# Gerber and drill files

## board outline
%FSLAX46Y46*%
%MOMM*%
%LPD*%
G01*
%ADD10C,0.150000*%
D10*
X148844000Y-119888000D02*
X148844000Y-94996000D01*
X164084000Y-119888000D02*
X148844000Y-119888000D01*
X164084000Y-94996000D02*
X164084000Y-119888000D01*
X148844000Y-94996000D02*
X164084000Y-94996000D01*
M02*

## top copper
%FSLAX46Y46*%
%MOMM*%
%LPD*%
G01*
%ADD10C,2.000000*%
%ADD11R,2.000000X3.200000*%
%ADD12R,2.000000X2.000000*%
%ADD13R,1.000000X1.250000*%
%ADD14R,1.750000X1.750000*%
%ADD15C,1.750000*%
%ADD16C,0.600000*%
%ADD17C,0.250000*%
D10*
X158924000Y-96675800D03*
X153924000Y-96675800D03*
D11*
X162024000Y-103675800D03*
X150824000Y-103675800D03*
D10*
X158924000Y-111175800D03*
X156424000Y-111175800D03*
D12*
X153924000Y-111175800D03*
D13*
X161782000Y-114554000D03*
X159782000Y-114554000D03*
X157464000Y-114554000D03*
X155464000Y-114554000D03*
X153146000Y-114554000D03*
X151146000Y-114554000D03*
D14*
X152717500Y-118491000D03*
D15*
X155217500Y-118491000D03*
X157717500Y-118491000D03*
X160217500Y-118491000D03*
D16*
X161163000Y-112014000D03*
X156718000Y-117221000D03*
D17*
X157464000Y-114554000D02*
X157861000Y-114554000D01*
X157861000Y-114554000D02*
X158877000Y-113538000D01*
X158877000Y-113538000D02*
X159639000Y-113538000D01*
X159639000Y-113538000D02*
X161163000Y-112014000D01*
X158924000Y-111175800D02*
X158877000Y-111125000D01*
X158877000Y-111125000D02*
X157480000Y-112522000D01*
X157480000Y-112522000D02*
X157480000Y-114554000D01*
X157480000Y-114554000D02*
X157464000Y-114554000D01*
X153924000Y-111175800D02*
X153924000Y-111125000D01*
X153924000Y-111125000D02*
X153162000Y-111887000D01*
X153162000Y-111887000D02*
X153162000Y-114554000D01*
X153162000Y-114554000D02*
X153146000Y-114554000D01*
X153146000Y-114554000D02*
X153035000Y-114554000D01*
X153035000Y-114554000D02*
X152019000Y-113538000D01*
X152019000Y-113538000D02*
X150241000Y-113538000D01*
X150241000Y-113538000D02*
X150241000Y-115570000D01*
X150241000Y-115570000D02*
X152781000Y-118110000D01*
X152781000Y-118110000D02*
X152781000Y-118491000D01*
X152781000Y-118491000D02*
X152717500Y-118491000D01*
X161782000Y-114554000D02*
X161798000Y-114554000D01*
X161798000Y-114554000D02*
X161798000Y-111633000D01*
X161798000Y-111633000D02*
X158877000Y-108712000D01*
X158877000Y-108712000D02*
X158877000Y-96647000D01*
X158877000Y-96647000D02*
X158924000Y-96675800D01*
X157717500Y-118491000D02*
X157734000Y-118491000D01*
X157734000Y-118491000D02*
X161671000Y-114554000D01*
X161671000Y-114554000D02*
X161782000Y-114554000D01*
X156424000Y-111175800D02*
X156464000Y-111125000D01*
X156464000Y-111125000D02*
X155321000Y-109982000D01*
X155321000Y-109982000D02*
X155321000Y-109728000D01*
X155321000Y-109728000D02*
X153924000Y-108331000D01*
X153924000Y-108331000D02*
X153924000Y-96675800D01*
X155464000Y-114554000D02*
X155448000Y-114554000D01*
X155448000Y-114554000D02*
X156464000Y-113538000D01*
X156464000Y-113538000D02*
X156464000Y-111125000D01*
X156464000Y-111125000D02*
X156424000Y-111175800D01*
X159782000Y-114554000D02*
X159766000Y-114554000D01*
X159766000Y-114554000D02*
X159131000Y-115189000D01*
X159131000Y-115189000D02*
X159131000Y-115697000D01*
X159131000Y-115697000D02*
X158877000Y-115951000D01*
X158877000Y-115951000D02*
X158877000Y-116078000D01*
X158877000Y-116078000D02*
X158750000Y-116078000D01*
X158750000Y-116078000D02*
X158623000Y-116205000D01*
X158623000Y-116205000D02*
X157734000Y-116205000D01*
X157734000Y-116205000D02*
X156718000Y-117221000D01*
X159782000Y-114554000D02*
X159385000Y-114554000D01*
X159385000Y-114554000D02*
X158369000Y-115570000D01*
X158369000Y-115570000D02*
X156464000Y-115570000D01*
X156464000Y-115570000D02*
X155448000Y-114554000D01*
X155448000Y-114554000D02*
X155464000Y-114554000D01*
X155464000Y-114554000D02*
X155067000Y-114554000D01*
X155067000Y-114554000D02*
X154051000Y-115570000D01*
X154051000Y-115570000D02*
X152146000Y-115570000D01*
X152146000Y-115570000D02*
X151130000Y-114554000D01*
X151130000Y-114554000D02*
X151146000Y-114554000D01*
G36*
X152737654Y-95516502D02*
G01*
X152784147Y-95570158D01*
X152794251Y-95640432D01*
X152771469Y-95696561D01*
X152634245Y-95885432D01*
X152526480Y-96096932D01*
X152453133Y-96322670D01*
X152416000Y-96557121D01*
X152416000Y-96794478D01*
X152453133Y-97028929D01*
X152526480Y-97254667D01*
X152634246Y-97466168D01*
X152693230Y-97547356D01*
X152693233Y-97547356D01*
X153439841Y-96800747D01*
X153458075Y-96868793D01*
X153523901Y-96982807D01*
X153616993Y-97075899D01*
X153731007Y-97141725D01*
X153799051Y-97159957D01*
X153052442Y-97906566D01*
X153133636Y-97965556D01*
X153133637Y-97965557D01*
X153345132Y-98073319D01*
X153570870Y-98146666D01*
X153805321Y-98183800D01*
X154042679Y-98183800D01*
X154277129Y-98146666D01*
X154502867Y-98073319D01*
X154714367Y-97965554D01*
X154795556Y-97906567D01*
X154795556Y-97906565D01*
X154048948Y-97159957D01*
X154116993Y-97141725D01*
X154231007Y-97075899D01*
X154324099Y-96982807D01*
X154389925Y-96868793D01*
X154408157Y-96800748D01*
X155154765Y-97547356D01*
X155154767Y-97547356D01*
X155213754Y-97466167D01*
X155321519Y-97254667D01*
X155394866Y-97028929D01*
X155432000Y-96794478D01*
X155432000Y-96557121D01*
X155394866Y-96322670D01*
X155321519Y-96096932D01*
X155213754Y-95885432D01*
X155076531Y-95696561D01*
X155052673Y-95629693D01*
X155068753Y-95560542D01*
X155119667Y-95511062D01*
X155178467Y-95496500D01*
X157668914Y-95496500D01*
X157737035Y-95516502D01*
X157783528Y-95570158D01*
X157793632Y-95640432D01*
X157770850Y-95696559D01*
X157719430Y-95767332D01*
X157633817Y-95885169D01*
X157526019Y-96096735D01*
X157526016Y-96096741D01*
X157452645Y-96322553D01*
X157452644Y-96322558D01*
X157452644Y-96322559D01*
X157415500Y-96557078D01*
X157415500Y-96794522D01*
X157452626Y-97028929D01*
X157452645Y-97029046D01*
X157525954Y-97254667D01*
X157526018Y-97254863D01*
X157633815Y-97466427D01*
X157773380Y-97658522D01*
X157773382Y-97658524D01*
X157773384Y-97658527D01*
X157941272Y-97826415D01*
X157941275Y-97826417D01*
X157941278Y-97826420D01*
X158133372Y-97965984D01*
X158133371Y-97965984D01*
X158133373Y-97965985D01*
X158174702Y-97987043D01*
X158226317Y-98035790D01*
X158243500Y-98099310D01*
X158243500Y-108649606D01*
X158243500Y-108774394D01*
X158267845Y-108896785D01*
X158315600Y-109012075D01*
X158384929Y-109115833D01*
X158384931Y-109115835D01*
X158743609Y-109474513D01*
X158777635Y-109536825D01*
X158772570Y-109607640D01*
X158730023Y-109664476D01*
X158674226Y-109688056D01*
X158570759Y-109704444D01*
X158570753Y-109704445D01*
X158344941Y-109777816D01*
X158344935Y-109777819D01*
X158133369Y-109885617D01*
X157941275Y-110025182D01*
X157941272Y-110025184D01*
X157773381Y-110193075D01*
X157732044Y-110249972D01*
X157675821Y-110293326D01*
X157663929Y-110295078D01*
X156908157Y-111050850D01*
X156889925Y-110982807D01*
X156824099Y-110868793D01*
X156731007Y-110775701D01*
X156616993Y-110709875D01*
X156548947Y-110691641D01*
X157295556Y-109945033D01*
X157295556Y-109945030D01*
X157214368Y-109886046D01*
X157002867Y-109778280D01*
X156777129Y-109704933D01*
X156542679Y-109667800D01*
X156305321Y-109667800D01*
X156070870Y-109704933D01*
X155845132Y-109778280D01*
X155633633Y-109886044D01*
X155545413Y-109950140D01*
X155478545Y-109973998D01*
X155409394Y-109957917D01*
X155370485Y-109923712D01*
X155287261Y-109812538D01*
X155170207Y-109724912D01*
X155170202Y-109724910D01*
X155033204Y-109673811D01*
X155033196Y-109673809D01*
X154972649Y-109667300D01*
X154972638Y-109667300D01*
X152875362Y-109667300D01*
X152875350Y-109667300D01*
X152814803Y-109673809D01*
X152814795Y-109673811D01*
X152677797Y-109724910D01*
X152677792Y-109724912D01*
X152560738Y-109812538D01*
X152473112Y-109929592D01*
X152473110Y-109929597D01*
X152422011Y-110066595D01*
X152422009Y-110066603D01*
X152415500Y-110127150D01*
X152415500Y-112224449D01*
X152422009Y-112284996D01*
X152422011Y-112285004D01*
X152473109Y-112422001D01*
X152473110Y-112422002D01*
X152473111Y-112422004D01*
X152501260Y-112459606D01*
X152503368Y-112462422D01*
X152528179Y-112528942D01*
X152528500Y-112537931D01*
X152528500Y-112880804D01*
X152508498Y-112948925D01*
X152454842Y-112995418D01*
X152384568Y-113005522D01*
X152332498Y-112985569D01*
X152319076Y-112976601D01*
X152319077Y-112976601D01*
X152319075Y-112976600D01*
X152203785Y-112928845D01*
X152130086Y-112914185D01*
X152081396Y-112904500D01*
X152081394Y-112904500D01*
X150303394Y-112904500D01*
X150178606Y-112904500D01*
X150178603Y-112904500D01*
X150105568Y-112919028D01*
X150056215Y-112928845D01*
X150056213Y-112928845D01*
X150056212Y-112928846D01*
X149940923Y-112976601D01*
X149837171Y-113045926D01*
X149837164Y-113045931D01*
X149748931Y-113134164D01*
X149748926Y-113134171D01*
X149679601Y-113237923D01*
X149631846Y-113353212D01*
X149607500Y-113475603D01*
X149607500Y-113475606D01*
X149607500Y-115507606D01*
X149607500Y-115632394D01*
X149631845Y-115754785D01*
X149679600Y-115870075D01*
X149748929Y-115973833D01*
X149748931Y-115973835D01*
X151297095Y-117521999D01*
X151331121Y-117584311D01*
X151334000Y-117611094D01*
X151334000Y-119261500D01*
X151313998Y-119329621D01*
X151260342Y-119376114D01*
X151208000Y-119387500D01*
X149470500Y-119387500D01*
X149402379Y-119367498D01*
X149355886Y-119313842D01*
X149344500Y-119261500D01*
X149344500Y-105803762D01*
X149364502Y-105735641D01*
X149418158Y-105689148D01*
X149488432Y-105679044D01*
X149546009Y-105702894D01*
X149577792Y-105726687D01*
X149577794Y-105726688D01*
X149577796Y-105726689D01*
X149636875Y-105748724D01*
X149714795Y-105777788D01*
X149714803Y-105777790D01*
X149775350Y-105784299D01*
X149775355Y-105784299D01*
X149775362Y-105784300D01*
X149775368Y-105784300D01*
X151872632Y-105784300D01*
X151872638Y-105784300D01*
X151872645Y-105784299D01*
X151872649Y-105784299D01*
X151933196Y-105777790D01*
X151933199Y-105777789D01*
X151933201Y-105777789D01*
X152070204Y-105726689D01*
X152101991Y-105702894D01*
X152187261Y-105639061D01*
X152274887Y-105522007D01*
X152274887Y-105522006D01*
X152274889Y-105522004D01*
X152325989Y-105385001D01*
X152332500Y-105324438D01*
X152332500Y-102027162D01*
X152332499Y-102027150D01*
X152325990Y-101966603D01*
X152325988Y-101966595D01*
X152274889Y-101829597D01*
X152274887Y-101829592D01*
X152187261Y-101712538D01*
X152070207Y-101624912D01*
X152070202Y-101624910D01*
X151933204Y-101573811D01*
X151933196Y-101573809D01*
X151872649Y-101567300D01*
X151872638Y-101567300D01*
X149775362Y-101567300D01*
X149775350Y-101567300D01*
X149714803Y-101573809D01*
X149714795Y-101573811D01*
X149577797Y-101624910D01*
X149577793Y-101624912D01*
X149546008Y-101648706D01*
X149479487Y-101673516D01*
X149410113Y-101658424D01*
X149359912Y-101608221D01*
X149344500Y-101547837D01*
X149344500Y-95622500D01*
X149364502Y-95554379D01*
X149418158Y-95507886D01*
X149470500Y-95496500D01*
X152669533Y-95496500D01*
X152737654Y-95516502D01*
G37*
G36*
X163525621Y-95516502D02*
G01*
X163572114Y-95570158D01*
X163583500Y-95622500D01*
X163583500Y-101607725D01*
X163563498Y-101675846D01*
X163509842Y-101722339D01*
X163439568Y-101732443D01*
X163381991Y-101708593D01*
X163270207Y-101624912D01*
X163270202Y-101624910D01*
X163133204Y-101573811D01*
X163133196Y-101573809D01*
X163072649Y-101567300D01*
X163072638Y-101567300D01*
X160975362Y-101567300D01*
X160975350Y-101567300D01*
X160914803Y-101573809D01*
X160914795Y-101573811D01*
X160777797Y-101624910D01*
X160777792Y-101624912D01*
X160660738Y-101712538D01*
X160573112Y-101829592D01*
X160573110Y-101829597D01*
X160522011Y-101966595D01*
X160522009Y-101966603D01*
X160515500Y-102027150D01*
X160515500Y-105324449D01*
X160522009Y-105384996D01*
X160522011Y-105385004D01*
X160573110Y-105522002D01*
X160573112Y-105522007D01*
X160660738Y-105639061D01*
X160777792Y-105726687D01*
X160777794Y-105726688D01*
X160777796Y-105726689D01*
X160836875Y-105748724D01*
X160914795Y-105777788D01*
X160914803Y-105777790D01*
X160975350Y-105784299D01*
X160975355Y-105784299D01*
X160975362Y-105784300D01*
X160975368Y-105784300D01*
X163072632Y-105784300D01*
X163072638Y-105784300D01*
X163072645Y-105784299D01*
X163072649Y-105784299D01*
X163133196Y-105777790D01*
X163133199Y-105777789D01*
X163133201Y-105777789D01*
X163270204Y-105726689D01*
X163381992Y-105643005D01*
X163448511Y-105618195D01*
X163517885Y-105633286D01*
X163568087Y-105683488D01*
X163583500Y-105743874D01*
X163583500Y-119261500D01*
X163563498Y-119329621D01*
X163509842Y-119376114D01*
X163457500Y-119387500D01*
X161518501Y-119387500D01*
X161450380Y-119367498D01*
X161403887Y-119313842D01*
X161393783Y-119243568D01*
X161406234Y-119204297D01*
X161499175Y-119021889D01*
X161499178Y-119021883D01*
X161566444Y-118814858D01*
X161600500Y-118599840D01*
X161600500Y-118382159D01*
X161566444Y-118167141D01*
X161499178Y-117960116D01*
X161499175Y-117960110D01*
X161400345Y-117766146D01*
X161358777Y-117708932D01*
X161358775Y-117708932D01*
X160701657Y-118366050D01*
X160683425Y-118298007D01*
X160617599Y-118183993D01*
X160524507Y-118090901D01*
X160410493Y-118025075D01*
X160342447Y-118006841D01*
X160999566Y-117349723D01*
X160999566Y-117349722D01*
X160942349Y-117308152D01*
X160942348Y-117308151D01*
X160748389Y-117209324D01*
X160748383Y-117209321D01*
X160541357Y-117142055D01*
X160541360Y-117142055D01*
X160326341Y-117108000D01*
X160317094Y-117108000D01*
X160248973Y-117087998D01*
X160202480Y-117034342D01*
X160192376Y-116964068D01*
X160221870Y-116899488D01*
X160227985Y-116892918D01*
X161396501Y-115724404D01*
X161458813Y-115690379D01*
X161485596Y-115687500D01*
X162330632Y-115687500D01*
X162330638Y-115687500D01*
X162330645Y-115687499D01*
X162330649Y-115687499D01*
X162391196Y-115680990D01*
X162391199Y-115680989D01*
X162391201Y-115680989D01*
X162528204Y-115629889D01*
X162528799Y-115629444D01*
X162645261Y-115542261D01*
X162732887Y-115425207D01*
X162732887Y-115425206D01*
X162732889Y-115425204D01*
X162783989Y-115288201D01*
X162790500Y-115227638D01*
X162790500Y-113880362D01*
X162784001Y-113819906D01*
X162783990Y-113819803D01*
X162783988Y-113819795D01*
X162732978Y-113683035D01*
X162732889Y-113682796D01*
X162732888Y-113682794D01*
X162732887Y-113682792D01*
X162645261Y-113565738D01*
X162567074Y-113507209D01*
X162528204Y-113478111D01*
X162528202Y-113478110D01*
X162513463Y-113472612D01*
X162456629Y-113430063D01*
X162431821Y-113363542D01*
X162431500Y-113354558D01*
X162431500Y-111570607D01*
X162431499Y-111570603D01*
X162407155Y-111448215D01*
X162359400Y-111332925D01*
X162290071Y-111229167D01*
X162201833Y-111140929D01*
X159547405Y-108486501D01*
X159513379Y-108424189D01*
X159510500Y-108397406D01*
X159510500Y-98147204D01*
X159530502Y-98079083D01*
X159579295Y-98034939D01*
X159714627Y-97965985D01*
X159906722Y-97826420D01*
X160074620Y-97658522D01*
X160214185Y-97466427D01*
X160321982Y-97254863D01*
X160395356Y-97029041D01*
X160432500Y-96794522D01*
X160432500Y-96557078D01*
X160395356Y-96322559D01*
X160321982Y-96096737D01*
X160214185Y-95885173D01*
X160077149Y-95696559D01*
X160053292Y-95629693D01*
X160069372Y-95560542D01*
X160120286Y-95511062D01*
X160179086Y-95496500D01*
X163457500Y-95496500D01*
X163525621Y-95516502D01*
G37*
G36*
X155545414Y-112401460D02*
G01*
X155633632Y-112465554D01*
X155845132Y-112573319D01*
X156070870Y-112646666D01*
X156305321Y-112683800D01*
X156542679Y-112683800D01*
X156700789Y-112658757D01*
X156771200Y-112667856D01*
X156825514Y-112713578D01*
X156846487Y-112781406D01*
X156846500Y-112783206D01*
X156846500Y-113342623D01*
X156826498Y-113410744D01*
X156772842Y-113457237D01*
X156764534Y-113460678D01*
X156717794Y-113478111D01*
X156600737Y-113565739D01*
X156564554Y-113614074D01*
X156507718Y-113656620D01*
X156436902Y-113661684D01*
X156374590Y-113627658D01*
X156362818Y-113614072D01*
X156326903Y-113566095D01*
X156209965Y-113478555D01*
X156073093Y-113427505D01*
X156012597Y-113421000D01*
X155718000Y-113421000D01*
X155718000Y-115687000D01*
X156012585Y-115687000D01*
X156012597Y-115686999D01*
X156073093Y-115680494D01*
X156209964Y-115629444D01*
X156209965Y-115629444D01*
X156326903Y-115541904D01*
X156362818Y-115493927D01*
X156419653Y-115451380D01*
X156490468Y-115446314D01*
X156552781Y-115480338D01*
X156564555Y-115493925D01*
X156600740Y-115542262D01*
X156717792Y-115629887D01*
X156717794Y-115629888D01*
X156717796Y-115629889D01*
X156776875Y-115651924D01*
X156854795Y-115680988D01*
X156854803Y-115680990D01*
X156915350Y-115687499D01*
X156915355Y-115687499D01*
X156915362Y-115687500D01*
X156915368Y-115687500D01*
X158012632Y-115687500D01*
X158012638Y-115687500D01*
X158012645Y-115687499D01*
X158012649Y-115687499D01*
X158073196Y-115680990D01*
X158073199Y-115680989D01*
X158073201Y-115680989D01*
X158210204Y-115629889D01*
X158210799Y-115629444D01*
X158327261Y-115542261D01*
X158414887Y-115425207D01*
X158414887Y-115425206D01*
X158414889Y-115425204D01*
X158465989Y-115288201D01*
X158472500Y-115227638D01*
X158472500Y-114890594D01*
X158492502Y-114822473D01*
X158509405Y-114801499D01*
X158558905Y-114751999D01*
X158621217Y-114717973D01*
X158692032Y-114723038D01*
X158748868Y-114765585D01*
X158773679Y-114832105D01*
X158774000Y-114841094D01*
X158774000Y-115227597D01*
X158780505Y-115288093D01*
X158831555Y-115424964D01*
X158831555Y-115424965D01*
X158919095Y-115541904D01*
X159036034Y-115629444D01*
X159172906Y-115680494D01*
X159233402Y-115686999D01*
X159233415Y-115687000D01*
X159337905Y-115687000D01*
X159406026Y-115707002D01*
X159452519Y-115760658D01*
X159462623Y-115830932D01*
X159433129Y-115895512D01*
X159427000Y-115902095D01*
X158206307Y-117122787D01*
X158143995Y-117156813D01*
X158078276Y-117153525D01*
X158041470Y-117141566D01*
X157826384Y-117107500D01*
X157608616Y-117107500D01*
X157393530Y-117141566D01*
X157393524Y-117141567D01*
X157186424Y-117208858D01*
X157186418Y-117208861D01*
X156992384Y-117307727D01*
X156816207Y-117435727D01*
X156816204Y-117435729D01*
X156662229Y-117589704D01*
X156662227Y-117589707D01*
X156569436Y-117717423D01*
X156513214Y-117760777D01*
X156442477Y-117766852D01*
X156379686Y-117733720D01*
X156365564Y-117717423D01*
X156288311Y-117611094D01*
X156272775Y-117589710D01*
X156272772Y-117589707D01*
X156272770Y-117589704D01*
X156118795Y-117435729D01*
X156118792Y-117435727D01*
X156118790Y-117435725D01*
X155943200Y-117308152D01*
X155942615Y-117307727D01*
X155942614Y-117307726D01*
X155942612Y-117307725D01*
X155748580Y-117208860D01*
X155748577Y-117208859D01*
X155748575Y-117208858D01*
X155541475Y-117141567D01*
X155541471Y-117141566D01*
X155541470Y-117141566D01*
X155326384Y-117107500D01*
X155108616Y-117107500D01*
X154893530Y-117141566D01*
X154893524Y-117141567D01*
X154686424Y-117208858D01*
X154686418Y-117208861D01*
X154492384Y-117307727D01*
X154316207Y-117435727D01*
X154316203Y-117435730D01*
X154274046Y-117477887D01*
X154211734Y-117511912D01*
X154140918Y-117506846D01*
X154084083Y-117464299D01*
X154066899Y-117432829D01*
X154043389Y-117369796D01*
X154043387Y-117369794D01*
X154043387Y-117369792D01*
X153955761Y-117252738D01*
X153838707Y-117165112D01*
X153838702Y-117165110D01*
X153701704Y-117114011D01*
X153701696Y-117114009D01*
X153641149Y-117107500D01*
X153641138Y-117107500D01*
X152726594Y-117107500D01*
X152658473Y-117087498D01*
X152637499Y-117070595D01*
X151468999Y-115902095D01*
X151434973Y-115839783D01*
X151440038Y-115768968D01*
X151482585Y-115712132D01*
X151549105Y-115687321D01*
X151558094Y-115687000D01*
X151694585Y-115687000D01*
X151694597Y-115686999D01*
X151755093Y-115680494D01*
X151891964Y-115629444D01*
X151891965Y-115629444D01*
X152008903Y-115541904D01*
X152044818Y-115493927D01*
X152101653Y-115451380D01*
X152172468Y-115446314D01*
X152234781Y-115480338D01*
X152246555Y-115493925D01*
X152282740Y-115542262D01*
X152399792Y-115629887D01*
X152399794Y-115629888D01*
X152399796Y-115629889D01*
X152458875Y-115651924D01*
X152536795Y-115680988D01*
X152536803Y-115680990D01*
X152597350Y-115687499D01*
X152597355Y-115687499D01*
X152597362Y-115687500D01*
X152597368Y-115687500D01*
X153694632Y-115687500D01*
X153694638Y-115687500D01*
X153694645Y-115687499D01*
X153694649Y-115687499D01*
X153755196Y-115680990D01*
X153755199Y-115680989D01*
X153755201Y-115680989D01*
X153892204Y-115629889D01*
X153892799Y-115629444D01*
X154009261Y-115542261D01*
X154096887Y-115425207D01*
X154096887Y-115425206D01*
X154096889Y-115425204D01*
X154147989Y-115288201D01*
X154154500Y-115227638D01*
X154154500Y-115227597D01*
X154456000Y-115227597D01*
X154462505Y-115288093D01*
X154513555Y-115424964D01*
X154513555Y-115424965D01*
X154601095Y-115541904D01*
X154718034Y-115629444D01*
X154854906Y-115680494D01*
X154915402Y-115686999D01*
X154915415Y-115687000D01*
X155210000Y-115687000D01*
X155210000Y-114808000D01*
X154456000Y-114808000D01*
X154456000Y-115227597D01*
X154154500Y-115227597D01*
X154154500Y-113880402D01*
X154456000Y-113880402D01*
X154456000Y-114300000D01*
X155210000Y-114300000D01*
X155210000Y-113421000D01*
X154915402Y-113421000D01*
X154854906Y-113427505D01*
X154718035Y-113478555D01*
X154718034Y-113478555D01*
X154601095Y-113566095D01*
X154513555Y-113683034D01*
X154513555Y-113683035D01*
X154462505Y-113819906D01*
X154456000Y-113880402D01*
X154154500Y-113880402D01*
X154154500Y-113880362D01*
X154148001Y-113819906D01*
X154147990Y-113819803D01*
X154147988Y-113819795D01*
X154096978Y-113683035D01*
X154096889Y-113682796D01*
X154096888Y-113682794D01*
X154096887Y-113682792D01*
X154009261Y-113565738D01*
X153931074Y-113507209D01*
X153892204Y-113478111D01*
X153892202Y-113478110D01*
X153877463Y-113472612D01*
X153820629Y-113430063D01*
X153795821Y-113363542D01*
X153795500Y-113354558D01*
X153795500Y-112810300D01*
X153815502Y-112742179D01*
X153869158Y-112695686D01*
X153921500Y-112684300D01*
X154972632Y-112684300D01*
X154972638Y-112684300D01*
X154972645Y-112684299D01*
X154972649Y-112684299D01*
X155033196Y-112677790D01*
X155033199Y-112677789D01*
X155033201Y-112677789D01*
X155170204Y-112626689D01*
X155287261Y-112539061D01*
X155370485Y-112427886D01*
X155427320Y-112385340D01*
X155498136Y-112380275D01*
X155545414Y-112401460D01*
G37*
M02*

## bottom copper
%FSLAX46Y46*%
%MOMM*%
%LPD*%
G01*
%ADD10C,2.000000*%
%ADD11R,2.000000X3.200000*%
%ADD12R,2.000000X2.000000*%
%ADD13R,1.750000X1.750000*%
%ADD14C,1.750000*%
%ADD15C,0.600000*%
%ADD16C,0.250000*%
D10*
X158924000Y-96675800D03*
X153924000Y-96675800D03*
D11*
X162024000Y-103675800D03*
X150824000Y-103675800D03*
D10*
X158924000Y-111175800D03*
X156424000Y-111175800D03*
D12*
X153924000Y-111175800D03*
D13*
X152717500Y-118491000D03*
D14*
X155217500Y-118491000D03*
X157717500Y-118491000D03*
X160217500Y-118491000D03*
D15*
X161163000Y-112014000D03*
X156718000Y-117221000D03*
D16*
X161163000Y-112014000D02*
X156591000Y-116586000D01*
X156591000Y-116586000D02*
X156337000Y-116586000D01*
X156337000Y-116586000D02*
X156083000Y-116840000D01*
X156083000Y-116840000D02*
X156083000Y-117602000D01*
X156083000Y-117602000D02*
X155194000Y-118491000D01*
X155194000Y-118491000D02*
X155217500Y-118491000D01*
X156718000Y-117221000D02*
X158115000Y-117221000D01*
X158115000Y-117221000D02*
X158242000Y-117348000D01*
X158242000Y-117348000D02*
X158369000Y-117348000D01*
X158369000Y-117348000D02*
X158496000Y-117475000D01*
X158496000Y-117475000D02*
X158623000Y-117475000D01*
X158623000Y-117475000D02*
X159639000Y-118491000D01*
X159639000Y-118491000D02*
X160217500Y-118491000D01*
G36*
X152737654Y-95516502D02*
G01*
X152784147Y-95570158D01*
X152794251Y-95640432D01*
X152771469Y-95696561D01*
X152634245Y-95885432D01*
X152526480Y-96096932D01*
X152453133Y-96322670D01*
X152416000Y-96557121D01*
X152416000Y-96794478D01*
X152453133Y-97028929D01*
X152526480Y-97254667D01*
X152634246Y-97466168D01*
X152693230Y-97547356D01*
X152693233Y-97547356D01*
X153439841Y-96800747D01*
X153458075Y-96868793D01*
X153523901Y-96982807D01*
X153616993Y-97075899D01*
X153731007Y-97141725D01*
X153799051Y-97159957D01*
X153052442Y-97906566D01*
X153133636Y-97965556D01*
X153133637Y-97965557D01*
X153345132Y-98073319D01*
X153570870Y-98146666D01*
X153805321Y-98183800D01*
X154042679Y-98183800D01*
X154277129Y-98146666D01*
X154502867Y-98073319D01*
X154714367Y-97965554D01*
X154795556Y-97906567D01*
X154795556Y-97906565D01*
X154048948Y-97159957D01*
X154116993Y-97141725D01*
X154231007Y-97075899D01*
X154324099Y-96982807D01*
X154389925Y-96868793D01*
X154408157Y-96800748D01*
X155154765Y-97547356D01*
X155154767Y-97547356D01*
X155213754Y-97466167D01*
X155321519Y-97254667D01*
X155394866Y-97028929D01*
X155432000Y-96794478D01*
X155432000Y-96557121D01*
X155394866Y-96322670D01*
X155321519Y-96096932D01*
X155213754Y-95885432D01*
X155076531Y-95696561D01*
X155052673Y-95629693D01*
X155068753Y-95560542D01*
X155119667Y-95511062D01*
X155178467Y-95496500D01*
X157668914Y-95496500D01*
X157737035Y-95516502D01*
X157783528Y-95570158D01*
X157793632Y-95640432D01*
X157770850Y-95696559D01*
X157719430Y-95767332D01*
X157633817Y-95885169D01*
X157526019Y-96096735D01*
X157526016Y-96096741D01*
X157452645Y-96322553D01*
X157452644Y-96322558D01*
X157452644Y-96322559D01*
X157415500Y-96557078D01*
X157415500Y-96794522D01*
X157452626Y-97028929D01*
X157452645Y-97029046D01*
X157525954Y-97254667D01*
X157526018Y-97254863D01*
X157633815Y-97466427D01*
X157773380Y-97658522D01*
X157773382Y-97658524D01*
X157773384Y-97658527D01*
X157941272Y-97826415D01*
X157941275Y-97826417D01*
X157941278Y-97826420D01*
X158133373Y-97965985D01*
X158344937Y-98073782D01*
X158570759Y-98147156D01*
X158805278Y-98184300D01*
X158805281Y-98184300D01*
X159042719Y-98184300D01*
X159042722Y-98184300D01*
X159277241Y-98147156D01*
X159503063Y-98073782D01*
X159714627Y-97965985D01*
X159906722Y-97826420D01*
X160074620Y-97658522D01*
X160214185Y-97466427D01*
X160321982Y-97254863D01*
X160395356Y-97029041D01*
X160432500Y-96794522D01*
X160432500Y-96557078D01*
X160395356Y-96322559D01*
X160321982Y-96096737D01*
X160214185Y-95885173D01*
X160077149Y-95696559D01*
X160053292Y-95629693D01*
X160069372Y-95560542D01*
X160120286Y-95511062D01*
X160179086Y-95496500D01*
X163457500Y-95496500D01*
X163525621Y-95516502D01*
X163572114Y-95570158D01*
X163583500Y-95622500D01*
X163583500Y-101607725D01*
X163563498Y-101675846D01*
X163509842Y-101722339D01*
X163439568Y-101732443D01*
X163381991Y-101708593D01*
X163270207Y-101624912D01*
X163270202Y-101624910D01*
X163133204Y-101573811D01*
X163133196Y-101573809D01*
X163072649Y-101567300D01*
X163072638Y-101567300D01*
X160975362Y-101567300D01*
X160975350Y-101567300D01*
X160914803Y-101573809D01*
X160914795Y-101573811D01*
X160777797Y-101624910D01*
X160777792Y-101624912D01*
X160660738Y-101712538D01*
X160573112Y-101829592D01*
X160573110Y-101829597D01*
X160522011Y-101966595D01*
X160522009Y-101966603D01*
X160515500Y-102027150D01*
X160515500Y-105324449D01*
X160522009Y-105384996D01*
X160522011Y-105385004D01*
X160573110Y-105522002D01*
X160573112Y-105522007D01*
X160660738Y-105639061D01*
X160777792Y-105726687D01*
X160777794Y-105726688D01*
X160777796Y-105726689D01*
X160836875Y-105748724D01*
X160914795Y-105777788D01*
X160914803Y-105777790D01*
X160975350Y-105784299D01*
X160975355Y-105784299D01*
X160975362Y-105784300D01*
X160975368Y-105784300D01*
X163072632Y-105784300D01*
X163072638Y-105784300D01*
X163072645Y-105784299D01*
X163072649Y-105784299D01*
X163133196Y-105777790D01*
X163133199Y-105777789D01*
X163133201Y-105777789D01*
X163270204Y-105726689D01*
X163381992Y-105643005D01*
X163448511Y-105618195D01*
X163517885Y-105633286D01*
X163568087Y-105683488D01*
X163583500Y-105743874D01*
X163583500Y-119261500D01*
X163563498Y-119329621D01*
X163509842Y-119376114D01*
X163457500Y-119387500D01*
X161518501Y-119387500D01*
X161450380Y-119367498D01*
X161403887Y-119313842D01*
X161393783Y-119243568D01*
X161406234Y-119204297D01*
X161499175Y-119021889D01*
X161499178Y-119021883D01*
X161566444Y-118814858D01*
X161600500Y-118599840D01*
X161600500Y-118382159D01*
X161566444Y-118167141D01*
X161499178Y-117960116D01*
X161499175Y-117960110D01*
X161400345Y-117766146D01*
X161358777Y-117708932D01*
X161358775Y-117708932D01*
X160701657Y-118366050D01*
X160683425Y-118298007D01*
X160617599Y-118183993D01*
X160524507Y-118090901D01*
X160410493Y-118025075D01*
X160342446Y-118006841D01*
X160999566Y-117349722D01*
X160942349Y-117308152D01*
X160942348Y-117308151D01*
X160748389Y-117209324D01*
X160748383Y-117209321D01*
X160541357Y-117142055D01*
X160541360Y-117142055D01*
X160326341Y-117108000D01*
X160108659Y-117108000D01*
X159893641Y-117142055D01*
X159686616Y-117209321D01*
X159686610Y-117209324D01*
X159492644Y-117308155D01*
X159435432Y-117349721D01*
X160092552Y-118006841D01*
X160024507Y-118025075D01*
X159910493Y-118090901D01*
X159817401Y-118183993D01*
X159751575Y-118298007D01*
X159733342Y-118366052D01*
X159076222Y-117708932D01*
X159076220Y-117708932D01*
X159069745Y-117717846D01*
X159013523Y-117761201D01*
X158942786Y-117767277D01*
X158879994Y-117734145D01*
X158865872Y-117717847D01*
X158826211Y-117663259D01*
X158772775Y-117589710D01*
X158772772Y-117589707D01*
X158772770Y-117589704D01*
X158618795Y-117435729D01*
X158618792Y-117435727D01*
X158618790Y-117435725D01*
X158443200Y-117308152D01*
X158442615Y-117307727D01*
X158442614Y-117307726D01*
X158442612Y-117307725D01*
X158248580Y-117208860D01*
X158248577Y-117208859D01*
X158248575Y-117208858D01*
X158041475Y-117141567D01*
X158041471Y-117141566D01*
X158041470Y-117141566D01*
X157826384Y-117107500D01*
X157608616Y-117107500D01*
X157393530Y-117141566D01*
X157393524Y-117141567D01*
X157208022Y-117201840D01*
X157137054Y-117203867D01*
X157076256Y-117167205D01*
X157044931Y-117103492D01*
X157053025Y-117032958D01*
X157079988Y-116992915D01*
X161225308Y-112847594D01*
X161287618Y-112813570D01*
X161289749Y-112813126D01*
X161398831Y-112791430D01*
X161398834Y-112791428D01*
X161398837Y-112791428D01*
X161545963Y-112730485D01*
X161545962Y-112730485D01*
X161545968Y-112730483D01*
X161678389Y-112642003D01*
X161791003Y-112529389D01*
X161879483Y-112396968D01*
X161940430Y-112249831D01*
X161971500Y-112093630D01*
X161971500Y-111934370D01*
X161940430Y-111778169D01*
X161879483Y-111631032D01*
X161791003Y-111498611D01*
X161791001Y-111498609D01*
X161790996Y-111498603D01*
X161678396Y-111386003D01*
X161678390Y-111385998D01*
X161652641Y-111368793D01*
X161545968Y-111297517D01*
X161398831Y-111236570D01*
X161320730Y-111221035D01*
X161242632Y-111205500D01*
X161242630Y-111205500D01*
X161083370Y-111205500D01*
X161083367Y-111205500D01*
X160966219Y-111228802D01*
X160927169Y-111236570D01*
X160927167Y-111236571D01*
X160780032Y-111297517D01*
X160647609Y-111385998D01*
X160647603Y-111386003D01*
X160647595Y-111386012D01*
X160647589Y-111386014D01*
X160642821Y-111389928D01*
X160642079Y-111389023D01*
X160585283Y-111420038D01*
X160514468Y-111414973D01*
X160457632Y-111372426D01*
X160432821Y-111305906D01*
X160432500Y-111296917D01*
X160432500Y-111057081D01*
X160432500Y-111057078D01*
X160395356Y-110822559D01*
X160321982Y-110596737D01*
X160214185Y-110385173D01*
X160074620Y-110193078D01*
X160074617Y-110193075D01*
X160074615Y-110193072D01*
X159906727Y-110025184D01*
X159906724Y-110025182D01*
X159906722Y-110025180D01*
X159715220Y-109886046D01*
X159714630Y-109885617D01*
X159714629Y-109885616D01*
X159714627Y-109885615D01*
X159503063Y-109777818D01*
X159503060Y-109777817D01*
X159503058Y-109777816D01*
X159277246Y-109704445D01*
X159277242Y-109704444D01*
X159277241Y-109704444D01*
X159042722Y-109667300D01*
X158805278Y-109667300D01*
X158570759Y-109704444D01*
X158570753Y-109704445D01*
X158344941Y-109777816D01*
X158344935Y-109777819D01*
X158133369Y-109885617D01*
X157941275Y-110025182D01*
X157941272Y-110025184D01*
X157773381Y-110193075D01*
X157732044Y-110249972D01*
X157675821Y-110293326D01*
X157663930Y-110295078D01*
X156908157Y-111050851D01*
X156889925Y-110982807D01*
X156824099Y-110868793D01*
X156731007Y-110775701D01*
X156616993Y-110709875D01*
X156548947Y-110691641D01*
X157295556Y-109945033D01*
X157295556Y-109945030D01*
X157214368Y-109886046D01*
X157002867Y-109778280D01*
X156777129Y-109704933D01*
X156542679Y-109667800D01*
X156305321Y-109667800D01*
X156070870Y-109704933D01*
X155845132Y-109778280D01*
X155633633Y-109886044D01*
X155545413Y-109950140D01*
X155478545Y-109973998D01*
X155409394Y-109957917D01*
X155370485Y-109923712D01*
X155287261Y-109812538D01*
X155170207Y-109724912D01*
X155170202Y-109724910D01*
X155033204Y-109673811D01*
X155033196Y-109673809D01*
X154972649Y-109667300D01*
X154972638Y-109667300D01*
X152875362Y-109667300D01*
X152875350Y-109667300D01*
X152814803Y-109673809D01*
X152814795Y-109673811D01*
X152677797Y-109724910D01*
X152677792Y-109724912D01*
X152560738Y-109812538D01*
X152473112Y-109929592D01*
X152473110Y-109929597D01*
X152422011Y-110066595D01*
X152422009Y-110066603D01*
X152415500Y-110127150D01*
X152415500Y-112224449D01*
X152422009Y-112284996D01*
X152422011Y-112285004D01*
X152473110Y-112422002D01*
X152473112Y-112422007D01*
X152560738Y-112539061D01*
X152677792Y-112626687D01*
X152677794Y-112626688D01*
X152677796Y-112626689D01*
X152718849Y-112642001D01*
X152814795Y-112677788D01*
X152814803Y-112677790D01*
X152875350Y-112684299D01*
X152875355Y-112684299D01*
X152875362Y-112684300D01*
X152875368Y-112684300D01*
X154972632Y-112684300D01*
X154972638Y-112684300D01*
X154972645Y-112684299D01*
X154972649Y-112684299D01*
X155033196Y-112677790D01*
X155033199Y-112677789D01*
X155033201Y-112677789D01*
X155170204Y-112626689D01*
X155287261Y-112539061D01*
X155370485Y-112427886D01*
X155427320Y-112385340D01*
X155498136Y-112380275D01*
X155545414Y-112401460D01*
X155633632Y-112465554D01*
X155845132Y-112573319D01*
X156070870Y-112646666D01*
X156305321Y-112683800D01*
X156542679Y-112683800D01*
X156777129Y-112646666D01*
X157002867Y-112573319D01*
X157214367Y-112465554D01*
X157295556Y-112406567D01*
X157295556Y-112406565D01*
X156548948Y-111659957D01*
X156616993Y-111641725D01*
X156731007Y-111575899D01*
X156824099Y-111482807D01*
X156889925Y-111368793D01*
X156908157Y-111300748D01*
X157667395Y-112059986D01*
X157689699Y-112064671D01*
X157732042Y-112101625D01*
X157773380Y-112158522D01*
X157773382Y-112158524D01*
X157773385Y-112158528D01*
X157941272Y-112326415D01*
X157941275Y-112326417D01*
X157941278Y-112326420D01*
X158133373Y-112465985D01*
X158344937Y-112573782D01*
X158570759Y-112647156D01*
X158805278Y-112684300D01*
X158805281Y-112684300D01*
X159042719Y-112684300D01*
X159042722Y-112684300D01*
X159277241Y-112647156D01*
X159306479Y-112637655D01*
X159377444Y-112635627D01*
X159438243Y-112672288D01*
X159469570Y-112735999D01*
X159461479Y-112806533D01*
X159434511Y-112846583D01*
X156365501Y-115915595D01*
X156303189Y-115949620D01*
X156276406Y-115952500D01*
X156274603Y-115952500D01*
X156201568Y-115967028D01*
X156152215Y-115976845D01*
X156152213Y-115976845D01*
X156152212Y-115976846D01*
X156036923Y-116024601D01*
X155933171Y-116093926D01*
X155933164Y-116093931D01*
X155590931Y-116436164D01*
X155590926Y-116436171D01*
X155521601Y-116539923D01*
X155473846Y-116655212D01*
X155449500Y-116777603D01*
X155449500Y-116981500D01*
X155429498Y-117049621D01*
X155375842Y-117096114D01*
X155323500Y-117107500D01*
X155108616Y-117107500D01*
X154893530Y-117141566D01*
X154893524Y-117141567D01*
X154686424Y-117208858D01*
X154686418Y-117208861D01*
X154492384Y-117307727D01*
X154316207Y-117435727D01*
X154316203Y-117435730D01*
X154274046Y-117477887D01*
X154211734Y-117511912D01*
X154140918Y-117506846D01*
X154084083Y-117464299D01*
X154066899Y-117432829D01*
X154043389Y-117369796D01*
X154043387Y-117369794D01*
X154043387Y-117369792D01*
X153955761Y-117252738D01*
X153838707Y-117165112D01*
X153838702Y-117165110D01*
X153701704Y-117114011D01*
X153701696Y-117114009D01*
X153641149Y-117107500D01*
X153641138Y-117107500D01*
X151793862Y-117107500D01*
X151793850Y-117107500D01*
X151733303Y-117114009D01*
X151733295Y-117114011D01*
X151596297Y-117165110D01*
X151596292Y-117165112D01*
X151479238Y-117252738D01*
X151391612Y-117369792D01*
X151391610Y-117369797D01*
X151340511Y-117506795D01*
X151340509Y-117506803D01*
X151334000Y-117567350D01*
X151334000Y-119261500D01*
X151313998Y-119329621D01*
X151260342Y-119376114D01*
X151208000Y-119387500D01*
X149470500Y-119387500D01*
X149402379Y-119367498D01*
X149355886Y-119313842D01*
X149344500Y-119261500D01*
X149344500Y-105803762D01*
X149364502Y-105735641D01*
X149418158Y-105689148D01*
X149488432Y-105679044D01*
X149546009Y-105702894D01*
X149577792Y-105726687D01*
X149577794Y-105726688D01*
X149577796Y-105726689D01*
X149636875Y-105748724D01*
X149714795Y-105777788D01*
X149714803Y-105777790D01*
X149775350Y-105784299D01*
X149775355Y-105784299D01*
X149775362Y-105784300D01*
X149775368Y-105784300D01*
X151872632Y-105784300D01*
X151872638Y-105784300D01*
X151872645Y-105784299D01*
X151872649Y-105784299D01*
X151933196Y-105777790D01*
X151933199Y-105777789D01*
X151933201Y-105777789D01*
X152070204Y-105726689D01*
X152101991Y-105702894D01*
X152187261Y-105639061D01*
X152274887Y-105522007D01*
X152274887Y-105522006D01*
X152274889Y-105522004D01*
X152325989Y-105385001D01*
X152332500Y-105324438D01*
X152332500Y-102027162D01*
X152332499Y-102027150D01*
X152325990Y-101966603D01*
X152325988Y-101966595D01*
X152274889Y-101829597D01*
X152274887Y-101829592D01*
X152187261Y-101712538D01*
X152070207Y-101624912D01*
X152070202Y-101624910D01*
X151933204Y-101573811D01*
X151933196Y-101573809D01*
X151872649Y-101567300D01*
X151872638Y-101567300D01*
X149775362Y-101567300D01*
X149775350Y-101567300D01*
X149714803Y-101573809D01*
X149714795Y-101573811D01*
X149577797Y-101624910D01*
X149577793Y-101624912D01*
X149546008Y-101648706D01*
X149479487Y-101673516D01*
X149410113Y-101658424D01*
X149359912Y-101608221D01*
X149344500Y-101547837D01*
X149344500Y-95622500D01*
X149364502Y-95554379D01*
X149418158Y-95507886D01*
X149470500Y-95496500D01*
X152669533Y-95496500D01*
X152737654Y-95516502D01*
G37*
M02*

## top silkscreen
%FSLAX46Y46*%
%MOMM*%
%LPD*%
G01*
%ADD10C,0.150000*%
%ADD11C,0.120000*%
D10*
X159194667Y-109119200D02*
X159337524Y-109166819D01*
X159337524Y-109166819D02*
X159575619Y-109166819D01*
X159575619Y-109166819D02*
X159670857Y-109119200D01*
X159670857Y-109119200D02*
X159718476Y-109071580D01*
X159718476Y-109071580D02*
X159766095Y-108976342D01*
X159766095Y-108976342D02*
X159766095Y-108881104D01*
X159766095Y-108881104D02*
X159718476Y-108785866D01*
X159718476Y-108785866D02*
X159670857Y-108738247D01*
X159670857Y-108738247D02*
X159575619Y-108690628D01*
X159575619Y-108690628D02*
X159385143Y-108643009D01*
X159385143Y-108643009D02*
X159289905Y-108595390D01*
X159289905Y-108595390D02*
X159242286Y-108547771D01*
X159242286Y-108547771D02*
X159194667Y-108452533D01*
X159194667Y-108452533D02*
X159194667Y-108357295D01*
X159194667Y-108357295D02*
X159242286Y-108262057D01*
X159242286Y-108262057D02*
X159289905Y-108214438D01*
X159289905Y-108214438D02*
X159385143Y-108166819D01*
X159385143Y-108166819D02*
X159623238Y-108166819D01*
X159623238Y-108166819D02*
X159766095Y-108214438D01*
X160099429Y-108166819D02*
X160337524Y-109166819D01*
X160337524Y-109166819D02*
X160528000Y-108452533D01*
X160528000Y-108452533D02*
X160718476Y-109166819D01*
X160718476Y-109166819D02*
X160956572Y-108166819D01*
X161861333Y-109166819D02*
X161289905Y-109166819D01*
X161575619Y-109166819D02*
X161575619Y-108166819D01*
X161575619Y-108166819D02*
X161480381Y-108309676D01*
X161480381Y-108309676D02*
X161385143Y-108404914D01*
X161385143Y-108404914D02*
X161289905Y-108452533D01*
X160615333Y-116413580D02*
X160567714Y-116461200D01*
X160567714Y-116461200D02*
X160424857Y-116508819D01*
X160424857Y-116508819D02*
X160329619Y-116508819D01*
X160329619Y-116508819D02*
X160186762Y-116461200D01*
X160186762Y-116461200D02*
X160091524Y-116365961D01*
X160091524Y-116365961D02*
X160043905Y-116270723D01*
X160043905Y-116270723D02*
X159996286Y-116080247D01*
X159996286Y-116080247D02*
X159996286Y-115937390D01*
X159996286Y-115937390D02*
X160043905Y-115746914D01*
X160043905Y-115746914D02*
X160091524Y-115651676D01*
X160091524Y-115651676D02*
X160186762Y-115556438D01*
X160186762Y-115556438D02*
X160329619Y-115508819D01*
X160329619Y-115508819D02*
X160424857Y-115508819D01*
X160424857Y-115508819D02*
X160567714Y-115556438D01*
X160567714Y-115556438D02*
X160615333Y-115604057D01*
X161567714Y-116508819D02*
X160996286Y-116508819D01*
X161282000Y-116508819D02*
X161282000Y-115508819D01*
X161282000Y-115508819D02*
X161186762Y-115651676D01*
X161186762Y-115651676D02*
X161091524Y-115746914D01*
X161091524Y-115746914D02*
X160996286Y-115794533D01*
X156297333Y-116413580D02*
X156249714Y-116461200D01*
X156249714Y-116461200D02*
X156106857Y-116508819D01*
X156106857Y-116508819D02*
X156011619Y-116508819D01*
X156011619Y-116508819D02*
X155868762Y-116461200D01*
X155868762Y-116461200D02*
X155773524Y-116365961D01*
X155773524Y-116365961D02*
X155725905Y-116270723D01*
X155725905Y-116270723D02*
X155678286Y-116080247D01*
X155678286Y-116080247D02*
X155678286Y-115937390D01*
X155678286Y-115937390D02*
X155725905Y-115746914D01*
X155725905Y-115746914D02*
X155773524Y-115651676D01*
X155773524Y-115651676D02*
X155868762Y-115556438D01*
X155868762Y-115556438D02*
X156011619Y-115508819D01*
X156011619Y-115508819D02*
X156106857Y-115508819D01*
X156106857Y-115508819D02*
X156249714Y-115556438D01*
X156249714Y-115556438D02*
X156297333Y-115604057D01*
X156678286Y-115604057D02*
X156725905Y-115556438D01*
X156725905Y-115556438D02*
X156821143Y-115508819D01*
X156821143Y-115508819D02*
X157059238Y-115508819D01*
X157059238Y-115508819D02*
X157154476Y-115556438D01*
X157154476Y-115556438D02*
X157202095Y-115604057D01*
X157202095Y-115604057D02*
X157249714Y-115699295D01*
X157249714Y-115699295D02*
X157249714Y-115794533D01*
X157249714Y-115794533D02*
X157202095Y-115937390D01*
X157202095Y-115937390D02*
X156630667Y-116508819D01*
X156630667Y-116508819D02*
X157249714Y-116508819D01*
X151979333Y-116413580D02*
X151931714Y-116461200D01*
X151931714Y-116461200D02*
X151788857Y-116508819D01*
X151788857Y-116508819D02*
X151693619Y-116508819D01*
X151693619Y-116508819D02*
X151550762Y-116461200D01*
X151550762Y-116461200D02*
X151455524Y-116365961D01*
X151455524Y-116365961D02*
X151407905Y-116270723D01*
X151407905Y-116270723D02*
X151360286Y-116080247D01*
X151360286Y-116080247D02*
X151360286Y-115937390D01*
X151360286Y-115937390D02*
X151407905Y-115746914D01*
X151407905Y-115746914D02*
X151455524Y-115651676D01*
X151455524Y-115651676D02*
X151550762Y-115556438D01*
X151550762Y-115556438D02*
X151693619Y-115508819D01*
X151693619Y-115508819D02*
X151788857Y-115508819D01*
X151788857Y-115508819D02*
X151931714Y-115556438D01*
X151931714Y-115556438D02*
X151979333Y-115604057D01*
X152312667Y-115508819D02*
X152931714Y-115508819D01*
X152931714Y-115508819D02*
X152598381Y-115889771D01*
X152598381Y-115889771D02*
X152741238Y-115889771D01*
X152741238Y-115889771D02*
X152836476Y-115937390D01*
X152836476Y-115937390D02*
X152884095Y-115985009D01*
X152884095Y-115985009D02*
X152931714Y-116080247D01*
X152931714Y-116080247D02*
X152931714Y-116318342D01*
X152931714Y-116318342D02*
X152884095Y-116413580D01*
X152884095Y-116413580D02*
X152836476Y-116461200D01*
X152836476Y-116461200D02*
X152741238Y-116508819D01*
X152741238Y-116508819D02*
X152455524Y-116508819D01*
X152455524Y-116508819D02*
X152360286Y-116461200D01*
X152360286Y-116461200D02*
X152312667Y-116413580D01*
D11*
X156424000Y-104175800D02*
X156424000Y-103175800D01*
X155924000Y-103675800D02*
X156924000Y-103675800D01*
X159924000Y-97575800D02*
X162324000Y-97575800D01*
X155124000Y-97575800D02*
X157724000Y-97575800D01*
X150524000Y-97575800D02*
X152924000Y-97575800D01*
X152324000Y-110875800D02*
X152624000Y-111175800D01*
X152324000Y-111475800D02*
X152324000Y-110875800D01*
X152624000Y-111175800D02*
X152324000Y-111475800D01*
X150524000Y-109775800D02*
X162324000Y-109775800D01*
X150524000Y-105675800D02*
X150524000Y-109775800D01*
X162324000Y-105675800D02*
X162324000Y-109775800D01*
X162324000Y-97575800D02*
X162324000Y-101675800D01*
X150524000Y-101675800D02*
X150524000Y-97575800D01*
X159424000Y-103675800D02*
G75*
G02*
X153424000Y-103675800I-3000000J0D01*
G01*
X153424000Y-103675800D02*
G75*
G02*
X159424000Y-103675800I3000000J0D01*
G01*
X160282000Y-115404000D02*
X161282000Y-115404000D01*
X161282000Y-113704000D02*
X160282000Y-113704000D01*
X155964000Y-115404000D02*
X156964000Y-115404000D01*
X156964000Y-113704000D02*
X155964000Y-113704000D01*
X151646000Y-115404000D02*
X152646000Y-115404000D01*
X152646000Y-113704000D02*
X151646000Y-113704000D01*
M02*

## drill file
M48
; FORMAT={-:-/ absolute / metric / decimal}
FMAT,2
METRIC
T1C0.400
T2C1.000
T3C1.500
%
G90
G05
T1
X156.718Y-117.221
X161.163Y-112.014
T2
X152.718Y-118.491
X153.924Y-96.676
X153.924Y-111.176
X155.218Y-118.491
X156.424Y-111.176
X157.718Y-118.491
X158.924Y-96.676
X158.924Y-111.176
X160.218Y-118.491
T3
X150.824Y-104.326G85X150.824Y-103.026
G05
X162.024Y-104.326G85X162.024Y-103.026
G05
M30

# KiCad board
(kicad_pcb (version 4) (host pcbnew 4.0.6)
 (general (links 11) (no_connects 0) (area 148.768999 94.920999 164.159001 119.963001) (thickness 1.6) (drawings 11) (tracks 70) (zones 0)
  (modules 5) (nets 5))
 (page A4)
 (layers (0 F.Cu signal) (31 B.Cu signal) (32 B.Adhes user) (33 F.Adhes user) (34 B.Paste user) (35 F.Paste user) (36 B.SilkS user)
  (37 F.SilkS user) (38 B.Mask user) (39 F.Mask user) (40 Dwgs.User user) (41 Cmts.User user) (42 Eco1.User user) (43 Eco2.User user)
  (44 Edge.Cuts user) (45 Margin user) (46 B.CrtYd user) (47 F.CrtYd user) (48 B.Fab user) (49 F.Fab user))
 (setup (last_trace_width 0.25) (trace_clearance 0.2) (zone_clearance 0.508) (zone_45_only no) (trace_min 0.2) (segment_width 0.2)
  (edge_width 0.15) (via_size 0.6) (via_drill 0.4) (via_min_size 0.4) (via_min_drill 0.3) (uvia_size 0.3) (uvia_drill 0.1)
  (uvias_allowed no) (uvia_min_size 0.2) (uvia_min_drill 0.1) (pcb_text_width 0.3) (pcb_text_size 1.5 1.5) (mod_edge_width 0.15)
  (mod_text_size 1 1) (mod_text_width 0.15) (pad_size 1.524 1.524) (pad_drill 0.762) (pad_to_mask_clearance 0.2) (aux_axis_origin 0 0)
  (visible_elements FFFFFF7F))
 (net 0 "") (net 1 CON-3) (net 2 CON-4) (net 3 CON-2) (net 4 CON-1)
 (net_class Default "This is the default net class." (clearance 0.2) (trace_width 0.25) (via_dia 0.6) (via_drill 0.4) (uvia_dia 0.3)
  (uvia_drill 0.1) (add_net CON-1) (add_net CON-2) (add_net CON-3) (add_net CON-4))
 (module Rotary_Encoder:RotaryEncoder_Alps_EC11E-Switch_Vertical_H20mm (layer F.Cu) (at 153.924 111.1758 90)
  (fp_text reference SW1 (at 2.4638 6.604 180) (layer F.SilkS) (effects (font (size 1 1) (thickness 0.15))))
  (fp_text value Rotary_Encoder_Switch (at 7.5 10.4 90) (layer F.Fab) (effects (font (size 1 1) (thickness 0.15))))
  (fp_line (start 7 2.5) (end 8 2.5) (layer F.SilkS) (width 0.12))
  (fp_line (start 7.5 2) (end 7.5 3) (layer F.SilkS) (width 0.12))
  (fp_line (start 13.6 6) (end 13.6 8.4) (layer F.SilkS) (width 0.12))
  (fp_line (start 13.6 1.2) (end 13.6 3.8) (layer F.SilkS) (width 0.12))
  (fp_line (start 13.6 -3.4) (end 13.6 -1) (layer F.SilkS) (width 0.12))
  (fp_line (start 0.3 -1.6) (end 0 -1.3) (layer F.SilkS) (width 0.12))
  (fp_line (start -0.3 -1.6) (end 0.3 -1.6) (layer F.SilkS) (width 0.12))
  (fp_line (start 0 -1.3) (end -0.3 -1.6) (layer F.SilkS) (width 0.12))
  (fp_line (start 1.4 -3.4) (end 1.4 8.4) (layer F.SilkS) (width 0.12))
  (fp_line (start 5.5 -3.4) (end 1.4 -3.4) (layer F.SilkS) (width 0.12))
  (fp_line (start 5.5 8.4) (end 1.4 8.4) (layer F.SilkS) (width 0.12))
  (fp_line (start 13.6 8.4) (end 9.5 8.4) (layer F.SilkS) (width 0.12))
  (fp_line (start 9.5 -3.4) (end 13.6 -3.4) (layer F.SilkS) (width 0.12))
  (fp_circle (center 7.5 2.5) (end 10.5 2.5) (layer F.SilkS) (width 0.12))
  (pad 4 thru_hole circle (at 14.5 5 90) (size 2 2) (drill 1) (layers *.Cu *.Mask) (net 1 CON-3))
  (pad 5 thru_hole circle (at 14.5 0 90) (size 2 2) (drill 1) (layers *.Cu *.Mask) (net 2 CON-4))
  (pad MP thru_hole rect (at 7.5 8.1 90) (size 3.2 2) (drill oval 2.8 1.5) (layers *.Cu *.Mask))
  (pad MP thru_hole rect (at 7.5 -3.1 90) (size 3.2 2) (drill oval 2.8 1.5) (layers *.Cu *.Mask))
  (pad 3 thru_hole circle (at 0 5 90) (size 2 2) (drill 1) (layers *.Cu *.Mask) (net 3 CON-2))
  (pad 2 thru_hole circle (at 0 2.5 90) (size 2 2) (drill 1) (layers *.Cu *.Mask) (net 2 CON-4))
  (pad 1 thru_hole rect (at 0 0 90) (size 2 2) (drill 1) (layers *.Cu *.Mask) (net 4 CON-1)))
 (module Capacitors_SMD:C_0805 (layer F.Cu) (at 160.782 114.554 180)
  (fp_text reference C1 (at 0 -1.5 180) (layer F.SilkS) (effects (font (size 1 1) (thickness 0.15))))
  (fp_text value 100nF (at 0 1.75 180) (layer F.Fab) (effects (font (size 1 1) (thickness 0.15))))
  (fp_line (start 0.5 -0.85) (end -0.5 -0.85) (layer F.SilkS) (width 0.12))
  (fp_line (start -0.5 0.85) (end 0.5 0.85) (layer F.SilkS) (width 0.12))
  (pad 1 smd rect (at -1 0 180) (size 1 1.25) (layers F.Cu F.Paste F.Mask) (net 1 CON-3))
  (pad 2 smd rect (at 1 0 180) (size 1 1.25) (layers F.Cu F.Paste F.Mask) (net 2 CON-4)))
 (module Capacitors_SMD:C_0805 (layer F.Cu) (at 156.464 114.554 180)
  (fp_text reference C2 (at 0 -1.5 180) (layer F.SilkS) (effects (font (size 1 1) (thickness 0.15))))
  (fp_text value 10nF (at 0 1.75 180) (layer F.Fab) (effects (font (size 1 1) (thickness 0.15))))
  (fp_line (start 0.5 -0.85) (end -0.5 -0.85) (layer F.SilkS) (width 0.12))
  (fp_line (start -0.5 0.85) (end 0.5 0.85) (layer F.SilkS) (width 0.12))
  (pad 1 smd rect (at -1 0 180) (size 1 1.25) (layers F.Cu F.Paste F.Mask) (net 3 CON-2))
  (pad 2 smd rect (at 1 0 180) (size 1 1.25) (layers F.Cu F.Paste F.Mask) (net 2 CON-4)))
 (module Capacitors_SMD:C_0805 (layer F.Cu) (at 152.146 114.554 180)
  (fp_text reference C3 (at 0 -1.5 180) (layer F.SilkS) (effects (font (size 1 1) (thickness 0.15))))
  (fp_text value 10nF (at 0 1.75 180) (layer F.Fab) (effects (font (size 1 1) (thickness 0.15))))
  (fp_line (start 0.5 -0.85) (end -0.5 -0.85) (layer F.SilkS) (width 0.12))
  (fp_line (start -0.5 0.85) (end 0.5 0.85) (layer F.SilkS) (width 0.12))
  (pad 1 smd rect (at -1 0 180) (size 1 1.25) (layers F.Cu F.Paste F.Mask) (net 4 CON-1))
  (pad 2 smd rect (at 1 0 180) (size 1 1.25) (layers F.Cu F.Paste F.Mask) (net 2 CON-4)))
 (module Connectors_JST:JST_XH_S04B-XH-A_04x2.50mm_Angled (layer B.Cu) (at 152.7175 118.491)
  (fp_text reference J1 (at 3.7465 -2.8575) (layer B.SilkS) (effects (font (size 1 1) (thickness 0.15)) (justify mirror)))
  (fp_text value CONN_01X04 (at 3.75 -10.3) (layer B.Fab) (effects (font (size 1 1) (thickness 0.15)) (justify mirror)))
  (pad 1 thru_hole rect (at 0 0) (size 1.75 1.75) (drill 1) (layers *.Cu *.Mask B.SilkS) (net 4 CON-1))
  (pad 2 thru_hole circle (at 2.5 0) (size 1.75 1.75) (drill 1) (layers *.Cu *.Mask B.SilkS) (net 3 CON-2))
  (pad 3 thru_hole circle (at 5 0) (size 1.75 1.75) (drill 1) (layers *.Cu *.Mask B.SilkS) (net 1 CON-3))
  (pad 4 thru_hole circle (at 7.5 0) (size 1.75 1.75) (drill 1) (layers *.Cu *.Mask B.SilkS) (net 2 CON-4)))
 (gr_line (start 148.844 119.888) (end 148.844 94.996) (angle 90) (layer Edge.Cuts) (width 0.15))
 (gr_line (start 164.084 119.888) (end 148.844 119.888) (angle 90) (layer Edge.Cuts) (width 0.15))
 (gr_line (start 164.084 94.996) (end 164.084 119.888) (angle 90) (layer Edge.Cuts) (width 0.15))
 (gr_line (start 148.844 94.996) (end 164.084 94.996) (angle 90) (layer Edge.Cuts) (width 0.15))
 (segment (start 157.464 114.554) (end 157.861 114.554) (width 0.25) (layer F.Cu) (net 3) (status 80000))
 (segment (start 157.861 114.554) (end 158.877 113.538) (width 0.25) (layer F.Cu) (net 3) (status 80000))
 (segment (start 158.877 113.538) (end 159.639 113.538) (width 0.25) (layer F.Cu) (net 3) (status 80000))
 (segment (start 159.639 113.538) (end 161.163 112.014) (width 0.25) (layer F.Cu) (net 3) (status 80000))
 (via (at 161.163 112.014) (size 0.6) (layers F.Cu B.Cu) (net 3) (status 80000))
 (segment (start 161.163 112.014) (end 156.591 116.586) (width 0.25) (layer B.Cu) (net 3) (status 80000))
 (segment (start 156.591 116.586) (end 156.337 116.586) (width 0.25) (layer B.Cu) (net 3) (status 80000))
 (segment (start 156.337 116.586) (end 156.083 116.84) (width 0.25) (layer B.Cu) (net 3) (status 80000))
 (segment (start 156.083 116.84) (end 156.083 117.602) (width 0.25) (layer B.Cu) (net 3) (status 80000))
 (segment (start 156.083 117.602) (end 155.194 118.491) (width 0.25) (layer B.Cu) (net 3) (status 80000))
 (segment (start 155.194 118.491) (end 155.2175 118.491) (width 0.25) (layer B.Cu) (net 3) (status 80000))
 (segment (start 158.924 111.1758) (end 158.877 111.125) (width 0.25) (layer F.Cu) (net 3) (status 80000))
 (segment (start 158.877 111.125) (end 157.48 112.522) (width 0.25) (layer F.Cu) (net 3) (status 80000))
 (segment (start 157.48 112.522) (end 157.48 114.554) (width 0.25) (layer F.Cu) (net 3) (status 80000))
 (segment (start 157.48 114.554) (end 157.464 114.554) (width 0.25) (layer F.Cu) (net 3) (status 80000))
 (segment (start 153.924 111.1758) (end 153.924 111.125) (width 0.25) (layer F.Cu) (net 4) (status 80000))
 (segment (start 153.924 111.125) (end 153.162 111.887) (width 0.25) (layer F.Cu) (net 4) (status 80000))
 (segment (start 153.162 111.887) (end 153.162 114.554) (width 0.25) (layer F.Cu) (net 4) (status 80000))
 (segment (start 153.162 114.554) (end 153.146 114.554) (width 0.25) (layer F.Cu) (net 4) (status 80000))
 (segment (start 153.146 114.554) (end 153.035 114.554) (width 0.25) (layer F.Cu) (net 4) (status 80000))
 (segment (start 153.035 114.554) (end 152.019 113.538) (width 0.25) (layer F.Cu) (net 4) (status 80000))
 (segment (start 152.019 113.538) (end 150.241 113.538) (width 0.25) (layer F.Cu) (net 4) (status 80000))
 (segment (start 150.241 113.538) (end 150.241 115.57) (width 0.25) (layer F.Cu) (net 4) (status 80000))
 (segment (start 150.241 115.57) (end 152.781 118.11) (width 0.25) (layer F.Cu) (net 4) (status 80000))
 (segment (start 152.781 118.11) (end 152.781 118.491) (width 0.25) (layer F.Cu) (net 4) (status 80000))
 (segment (start 152.781 118.491) (end 152.7175 118.491) (width 0.25) (layer F.Cu) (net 4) (status 80000))
 (segment (start 161.782 114.554) (end 161.798 114.554) (width 0.25) (layer F.Cu) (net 1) (status 80000))
 (segment (start 161.798 114.554) (end 161.798 111.633) (width 0.25) (layer F.Cu) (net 1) (status 80000))
 (segment (start 161.798 111.633) (end 158.877 108.712) (width 0.25) (layer F.Cu) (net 1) (status 80000))
 (segment (start 158.877 108.712) (end 158.877 96.647) (width 0.25) (layer F.Cu) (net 1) (status 80000))
 (segment (start 158.877 96.647) (end 158.924 96.6758) (width 0.25) (layer F.Cu) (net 1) (status 80000))
 (segment (start 157.7175 118.491) (end 157.734 118.491) (width 0.25) (layer F.Cu) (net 1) (status 80000))
 (segment (start 157.734 118.491) (end 161.671 114.554) (width 0.25) (layer F.Cu) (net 1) (status 80000))
 (segment (start 161.671 114.554) (end 161.782 114.554) (width 0.25) (layer F.Cu) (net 1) (status 80000))
 (segment (start 156.424 111.1758) (end 156.464 111.125) (width 0.25) (layer F.Cu) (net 2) (status 80000))
 (segment (start 156.464 111.125) (end 155.321 109.982) (width 0.25) (layer F.Cu) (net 2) (status 80000))
 (segment (start 155.321 109.982) (end 155.321 109.728) (width 0.25) (layer F.Cu) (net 2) (status 80000))
 (segment (start 155.321 109.728) (end 153.924 108.331) (width 0.25) (layer F.Cu) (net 2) (status 80000))
 (segment (start 153.924 108.331) (end 153.924 96.6758) (width 0.25) (layer F.Cu) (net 2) (status 80000))
 (segment (start 155.464 114.554) (end 155.448 114.554) (width 0.25) (layer F.Cu) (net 2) (status 80000))
 (segment (start 155.448 114.554) (end 156.464 113.538) (width 0.25) (layer F.Cu) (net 2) (status 80000))
 (segment (start 156.464 113.538) (end 156.464 111.125) (width 0.25) (layer F.Cu) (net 2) (status 80000))
 (segment (start 156.464 111.125) (end 156.424 111.1758) (width 0.25) (layer F.Cu) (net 2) (status 80000))
 (segment (start 159.782 114.554) (end 159.766 114.554) (width 0.25) (layer F.Cu) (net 2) (status 80000))
 (segment (start 159.766 114.554) (end 159.131 115.189) (width 0.25) (layer F.Cu) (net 2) (status 80000))
 (segment (start 159.131 115.189) (end 159.131 115.697) (width 0.25) (layer F.Cu) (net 2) (status 80000))
 (segment (start 159.131 115.697) (end 158.877 115.951) (width 0.25) (layer F.Cu) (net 2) (status 80000))
 (segment (start 158.877 115.951) (end 158.877 116.078) (width 0.25) (layer F.Cu) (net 2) (status 80000))
 (segment (start 158.877 116.078) (end 158.75 116.078) (width 0.25) (layer F.Cu) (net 2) (status 80000))
 (segment (start 158.75 116.078) (end 158.623 116.205) (width 0.25) (layer F.Cu) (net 2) (status 80000))
 (segment (start 158.623 116.205) (end 157.734 116.205) (width 0.25) (layer F.Cu) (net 2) (status 80000))
 (segment (start 157.734 116.205) (end 156.718 117.221) (width 0.25) (layer F.Cu) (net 2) (status 80000))
 (via (at 156.718 117.221) (size 0.6) (layers F.Cu B.Cu) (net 2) (status 80000))
 (segment (start 156.718 117.221) (end 158.115 117.221) (width 0.25) (layer B.Cu) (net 2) (status 80000))
 (segment (start 158.115 117.221) (end 158.242 117.348) (width 0.25) (layer B.Cu) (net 2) (status 80000))
 (segment (start 158.242 117.348) (end 158.369 117.348) (width 0.25) (layer B.Cu) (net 2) (status 80000))
 (segment (start 158.369 117.348) (end 158.496 117.475) (width 0.25) (layer B.Cu) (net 2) (status 80000))
 (segment (start 158.496 117.475) (end 158.623 117.475) (width 0.25) (layer B.Cu) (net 2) (status 80000))
 (segment (start 158.623 117.475) (end 159.639 118.491) (width 0.25) (layer B.Cu) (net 2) (status 80000))
 (segment (start 159.639 118.491) (end 160.2175 118.491) (width 0.25) (layer B.Cu) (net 2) (status 80000))
 (segment (start 159.782 114.554) (end 159.385 114.554) (width 0.25) (layer F.Cu) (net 2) (status 80000))
 (segment (start 159.385 114.554) (end 158.369 115.57) (width 0.25) (layer F.Cu) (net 2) (status 80000))
 (segment (start 158.369 115.57) (end 156.464 115.57) (width 0.25) (layer F.Cu) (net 2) (status 80000))
 (segment (start 156.464 115.57) (end 155.448 114.554) (width 0.25) (layer F.Cu) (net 2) (status 80000))
 (segment (start 155.448 114.554) (end 155.464 114.554) (width 0.25) (layer F.Cu) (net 2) (status 80000))
 (segment (start 155.464 114.554) (end 155.067 114.554) (width 0.25) (layer F.Cu) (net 2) (status 80000))
 (segment (start 155.067 114.554) (end 154.051 115.57) (width 0.25) (layer F.Cu) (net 2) (status 80000))
 (segment (start 154.051 115.57) (end 152.146 115.57) (width 0.25) (layer F.Cu) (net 2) (status 80000))
 (segment (start 152.146 115.57) (end 151.13 114.554) (width 0.25) (layer F.Cu) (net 2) (status 80000))
 (segment (start 151.13 114.554) (end 151.146 114.554) (width 0.25) (layer F.Cu) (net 2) (status 80000))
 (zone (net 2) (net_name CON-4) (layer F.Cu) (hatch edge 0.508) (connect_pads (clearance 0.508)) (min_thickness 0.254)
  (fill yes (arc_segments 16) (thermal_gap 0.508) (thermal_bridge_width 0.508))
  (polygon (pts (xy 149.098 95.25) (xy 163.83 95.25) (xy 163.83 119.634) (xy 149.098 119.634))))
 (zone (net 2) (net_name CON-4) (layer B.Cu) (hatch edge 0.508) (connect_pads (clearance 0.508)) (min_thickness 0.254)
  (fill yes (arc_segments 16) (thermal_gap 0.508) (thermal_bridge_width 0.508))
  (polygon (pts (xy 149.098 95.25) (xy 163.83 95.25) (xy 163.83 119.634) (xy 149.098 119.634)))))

